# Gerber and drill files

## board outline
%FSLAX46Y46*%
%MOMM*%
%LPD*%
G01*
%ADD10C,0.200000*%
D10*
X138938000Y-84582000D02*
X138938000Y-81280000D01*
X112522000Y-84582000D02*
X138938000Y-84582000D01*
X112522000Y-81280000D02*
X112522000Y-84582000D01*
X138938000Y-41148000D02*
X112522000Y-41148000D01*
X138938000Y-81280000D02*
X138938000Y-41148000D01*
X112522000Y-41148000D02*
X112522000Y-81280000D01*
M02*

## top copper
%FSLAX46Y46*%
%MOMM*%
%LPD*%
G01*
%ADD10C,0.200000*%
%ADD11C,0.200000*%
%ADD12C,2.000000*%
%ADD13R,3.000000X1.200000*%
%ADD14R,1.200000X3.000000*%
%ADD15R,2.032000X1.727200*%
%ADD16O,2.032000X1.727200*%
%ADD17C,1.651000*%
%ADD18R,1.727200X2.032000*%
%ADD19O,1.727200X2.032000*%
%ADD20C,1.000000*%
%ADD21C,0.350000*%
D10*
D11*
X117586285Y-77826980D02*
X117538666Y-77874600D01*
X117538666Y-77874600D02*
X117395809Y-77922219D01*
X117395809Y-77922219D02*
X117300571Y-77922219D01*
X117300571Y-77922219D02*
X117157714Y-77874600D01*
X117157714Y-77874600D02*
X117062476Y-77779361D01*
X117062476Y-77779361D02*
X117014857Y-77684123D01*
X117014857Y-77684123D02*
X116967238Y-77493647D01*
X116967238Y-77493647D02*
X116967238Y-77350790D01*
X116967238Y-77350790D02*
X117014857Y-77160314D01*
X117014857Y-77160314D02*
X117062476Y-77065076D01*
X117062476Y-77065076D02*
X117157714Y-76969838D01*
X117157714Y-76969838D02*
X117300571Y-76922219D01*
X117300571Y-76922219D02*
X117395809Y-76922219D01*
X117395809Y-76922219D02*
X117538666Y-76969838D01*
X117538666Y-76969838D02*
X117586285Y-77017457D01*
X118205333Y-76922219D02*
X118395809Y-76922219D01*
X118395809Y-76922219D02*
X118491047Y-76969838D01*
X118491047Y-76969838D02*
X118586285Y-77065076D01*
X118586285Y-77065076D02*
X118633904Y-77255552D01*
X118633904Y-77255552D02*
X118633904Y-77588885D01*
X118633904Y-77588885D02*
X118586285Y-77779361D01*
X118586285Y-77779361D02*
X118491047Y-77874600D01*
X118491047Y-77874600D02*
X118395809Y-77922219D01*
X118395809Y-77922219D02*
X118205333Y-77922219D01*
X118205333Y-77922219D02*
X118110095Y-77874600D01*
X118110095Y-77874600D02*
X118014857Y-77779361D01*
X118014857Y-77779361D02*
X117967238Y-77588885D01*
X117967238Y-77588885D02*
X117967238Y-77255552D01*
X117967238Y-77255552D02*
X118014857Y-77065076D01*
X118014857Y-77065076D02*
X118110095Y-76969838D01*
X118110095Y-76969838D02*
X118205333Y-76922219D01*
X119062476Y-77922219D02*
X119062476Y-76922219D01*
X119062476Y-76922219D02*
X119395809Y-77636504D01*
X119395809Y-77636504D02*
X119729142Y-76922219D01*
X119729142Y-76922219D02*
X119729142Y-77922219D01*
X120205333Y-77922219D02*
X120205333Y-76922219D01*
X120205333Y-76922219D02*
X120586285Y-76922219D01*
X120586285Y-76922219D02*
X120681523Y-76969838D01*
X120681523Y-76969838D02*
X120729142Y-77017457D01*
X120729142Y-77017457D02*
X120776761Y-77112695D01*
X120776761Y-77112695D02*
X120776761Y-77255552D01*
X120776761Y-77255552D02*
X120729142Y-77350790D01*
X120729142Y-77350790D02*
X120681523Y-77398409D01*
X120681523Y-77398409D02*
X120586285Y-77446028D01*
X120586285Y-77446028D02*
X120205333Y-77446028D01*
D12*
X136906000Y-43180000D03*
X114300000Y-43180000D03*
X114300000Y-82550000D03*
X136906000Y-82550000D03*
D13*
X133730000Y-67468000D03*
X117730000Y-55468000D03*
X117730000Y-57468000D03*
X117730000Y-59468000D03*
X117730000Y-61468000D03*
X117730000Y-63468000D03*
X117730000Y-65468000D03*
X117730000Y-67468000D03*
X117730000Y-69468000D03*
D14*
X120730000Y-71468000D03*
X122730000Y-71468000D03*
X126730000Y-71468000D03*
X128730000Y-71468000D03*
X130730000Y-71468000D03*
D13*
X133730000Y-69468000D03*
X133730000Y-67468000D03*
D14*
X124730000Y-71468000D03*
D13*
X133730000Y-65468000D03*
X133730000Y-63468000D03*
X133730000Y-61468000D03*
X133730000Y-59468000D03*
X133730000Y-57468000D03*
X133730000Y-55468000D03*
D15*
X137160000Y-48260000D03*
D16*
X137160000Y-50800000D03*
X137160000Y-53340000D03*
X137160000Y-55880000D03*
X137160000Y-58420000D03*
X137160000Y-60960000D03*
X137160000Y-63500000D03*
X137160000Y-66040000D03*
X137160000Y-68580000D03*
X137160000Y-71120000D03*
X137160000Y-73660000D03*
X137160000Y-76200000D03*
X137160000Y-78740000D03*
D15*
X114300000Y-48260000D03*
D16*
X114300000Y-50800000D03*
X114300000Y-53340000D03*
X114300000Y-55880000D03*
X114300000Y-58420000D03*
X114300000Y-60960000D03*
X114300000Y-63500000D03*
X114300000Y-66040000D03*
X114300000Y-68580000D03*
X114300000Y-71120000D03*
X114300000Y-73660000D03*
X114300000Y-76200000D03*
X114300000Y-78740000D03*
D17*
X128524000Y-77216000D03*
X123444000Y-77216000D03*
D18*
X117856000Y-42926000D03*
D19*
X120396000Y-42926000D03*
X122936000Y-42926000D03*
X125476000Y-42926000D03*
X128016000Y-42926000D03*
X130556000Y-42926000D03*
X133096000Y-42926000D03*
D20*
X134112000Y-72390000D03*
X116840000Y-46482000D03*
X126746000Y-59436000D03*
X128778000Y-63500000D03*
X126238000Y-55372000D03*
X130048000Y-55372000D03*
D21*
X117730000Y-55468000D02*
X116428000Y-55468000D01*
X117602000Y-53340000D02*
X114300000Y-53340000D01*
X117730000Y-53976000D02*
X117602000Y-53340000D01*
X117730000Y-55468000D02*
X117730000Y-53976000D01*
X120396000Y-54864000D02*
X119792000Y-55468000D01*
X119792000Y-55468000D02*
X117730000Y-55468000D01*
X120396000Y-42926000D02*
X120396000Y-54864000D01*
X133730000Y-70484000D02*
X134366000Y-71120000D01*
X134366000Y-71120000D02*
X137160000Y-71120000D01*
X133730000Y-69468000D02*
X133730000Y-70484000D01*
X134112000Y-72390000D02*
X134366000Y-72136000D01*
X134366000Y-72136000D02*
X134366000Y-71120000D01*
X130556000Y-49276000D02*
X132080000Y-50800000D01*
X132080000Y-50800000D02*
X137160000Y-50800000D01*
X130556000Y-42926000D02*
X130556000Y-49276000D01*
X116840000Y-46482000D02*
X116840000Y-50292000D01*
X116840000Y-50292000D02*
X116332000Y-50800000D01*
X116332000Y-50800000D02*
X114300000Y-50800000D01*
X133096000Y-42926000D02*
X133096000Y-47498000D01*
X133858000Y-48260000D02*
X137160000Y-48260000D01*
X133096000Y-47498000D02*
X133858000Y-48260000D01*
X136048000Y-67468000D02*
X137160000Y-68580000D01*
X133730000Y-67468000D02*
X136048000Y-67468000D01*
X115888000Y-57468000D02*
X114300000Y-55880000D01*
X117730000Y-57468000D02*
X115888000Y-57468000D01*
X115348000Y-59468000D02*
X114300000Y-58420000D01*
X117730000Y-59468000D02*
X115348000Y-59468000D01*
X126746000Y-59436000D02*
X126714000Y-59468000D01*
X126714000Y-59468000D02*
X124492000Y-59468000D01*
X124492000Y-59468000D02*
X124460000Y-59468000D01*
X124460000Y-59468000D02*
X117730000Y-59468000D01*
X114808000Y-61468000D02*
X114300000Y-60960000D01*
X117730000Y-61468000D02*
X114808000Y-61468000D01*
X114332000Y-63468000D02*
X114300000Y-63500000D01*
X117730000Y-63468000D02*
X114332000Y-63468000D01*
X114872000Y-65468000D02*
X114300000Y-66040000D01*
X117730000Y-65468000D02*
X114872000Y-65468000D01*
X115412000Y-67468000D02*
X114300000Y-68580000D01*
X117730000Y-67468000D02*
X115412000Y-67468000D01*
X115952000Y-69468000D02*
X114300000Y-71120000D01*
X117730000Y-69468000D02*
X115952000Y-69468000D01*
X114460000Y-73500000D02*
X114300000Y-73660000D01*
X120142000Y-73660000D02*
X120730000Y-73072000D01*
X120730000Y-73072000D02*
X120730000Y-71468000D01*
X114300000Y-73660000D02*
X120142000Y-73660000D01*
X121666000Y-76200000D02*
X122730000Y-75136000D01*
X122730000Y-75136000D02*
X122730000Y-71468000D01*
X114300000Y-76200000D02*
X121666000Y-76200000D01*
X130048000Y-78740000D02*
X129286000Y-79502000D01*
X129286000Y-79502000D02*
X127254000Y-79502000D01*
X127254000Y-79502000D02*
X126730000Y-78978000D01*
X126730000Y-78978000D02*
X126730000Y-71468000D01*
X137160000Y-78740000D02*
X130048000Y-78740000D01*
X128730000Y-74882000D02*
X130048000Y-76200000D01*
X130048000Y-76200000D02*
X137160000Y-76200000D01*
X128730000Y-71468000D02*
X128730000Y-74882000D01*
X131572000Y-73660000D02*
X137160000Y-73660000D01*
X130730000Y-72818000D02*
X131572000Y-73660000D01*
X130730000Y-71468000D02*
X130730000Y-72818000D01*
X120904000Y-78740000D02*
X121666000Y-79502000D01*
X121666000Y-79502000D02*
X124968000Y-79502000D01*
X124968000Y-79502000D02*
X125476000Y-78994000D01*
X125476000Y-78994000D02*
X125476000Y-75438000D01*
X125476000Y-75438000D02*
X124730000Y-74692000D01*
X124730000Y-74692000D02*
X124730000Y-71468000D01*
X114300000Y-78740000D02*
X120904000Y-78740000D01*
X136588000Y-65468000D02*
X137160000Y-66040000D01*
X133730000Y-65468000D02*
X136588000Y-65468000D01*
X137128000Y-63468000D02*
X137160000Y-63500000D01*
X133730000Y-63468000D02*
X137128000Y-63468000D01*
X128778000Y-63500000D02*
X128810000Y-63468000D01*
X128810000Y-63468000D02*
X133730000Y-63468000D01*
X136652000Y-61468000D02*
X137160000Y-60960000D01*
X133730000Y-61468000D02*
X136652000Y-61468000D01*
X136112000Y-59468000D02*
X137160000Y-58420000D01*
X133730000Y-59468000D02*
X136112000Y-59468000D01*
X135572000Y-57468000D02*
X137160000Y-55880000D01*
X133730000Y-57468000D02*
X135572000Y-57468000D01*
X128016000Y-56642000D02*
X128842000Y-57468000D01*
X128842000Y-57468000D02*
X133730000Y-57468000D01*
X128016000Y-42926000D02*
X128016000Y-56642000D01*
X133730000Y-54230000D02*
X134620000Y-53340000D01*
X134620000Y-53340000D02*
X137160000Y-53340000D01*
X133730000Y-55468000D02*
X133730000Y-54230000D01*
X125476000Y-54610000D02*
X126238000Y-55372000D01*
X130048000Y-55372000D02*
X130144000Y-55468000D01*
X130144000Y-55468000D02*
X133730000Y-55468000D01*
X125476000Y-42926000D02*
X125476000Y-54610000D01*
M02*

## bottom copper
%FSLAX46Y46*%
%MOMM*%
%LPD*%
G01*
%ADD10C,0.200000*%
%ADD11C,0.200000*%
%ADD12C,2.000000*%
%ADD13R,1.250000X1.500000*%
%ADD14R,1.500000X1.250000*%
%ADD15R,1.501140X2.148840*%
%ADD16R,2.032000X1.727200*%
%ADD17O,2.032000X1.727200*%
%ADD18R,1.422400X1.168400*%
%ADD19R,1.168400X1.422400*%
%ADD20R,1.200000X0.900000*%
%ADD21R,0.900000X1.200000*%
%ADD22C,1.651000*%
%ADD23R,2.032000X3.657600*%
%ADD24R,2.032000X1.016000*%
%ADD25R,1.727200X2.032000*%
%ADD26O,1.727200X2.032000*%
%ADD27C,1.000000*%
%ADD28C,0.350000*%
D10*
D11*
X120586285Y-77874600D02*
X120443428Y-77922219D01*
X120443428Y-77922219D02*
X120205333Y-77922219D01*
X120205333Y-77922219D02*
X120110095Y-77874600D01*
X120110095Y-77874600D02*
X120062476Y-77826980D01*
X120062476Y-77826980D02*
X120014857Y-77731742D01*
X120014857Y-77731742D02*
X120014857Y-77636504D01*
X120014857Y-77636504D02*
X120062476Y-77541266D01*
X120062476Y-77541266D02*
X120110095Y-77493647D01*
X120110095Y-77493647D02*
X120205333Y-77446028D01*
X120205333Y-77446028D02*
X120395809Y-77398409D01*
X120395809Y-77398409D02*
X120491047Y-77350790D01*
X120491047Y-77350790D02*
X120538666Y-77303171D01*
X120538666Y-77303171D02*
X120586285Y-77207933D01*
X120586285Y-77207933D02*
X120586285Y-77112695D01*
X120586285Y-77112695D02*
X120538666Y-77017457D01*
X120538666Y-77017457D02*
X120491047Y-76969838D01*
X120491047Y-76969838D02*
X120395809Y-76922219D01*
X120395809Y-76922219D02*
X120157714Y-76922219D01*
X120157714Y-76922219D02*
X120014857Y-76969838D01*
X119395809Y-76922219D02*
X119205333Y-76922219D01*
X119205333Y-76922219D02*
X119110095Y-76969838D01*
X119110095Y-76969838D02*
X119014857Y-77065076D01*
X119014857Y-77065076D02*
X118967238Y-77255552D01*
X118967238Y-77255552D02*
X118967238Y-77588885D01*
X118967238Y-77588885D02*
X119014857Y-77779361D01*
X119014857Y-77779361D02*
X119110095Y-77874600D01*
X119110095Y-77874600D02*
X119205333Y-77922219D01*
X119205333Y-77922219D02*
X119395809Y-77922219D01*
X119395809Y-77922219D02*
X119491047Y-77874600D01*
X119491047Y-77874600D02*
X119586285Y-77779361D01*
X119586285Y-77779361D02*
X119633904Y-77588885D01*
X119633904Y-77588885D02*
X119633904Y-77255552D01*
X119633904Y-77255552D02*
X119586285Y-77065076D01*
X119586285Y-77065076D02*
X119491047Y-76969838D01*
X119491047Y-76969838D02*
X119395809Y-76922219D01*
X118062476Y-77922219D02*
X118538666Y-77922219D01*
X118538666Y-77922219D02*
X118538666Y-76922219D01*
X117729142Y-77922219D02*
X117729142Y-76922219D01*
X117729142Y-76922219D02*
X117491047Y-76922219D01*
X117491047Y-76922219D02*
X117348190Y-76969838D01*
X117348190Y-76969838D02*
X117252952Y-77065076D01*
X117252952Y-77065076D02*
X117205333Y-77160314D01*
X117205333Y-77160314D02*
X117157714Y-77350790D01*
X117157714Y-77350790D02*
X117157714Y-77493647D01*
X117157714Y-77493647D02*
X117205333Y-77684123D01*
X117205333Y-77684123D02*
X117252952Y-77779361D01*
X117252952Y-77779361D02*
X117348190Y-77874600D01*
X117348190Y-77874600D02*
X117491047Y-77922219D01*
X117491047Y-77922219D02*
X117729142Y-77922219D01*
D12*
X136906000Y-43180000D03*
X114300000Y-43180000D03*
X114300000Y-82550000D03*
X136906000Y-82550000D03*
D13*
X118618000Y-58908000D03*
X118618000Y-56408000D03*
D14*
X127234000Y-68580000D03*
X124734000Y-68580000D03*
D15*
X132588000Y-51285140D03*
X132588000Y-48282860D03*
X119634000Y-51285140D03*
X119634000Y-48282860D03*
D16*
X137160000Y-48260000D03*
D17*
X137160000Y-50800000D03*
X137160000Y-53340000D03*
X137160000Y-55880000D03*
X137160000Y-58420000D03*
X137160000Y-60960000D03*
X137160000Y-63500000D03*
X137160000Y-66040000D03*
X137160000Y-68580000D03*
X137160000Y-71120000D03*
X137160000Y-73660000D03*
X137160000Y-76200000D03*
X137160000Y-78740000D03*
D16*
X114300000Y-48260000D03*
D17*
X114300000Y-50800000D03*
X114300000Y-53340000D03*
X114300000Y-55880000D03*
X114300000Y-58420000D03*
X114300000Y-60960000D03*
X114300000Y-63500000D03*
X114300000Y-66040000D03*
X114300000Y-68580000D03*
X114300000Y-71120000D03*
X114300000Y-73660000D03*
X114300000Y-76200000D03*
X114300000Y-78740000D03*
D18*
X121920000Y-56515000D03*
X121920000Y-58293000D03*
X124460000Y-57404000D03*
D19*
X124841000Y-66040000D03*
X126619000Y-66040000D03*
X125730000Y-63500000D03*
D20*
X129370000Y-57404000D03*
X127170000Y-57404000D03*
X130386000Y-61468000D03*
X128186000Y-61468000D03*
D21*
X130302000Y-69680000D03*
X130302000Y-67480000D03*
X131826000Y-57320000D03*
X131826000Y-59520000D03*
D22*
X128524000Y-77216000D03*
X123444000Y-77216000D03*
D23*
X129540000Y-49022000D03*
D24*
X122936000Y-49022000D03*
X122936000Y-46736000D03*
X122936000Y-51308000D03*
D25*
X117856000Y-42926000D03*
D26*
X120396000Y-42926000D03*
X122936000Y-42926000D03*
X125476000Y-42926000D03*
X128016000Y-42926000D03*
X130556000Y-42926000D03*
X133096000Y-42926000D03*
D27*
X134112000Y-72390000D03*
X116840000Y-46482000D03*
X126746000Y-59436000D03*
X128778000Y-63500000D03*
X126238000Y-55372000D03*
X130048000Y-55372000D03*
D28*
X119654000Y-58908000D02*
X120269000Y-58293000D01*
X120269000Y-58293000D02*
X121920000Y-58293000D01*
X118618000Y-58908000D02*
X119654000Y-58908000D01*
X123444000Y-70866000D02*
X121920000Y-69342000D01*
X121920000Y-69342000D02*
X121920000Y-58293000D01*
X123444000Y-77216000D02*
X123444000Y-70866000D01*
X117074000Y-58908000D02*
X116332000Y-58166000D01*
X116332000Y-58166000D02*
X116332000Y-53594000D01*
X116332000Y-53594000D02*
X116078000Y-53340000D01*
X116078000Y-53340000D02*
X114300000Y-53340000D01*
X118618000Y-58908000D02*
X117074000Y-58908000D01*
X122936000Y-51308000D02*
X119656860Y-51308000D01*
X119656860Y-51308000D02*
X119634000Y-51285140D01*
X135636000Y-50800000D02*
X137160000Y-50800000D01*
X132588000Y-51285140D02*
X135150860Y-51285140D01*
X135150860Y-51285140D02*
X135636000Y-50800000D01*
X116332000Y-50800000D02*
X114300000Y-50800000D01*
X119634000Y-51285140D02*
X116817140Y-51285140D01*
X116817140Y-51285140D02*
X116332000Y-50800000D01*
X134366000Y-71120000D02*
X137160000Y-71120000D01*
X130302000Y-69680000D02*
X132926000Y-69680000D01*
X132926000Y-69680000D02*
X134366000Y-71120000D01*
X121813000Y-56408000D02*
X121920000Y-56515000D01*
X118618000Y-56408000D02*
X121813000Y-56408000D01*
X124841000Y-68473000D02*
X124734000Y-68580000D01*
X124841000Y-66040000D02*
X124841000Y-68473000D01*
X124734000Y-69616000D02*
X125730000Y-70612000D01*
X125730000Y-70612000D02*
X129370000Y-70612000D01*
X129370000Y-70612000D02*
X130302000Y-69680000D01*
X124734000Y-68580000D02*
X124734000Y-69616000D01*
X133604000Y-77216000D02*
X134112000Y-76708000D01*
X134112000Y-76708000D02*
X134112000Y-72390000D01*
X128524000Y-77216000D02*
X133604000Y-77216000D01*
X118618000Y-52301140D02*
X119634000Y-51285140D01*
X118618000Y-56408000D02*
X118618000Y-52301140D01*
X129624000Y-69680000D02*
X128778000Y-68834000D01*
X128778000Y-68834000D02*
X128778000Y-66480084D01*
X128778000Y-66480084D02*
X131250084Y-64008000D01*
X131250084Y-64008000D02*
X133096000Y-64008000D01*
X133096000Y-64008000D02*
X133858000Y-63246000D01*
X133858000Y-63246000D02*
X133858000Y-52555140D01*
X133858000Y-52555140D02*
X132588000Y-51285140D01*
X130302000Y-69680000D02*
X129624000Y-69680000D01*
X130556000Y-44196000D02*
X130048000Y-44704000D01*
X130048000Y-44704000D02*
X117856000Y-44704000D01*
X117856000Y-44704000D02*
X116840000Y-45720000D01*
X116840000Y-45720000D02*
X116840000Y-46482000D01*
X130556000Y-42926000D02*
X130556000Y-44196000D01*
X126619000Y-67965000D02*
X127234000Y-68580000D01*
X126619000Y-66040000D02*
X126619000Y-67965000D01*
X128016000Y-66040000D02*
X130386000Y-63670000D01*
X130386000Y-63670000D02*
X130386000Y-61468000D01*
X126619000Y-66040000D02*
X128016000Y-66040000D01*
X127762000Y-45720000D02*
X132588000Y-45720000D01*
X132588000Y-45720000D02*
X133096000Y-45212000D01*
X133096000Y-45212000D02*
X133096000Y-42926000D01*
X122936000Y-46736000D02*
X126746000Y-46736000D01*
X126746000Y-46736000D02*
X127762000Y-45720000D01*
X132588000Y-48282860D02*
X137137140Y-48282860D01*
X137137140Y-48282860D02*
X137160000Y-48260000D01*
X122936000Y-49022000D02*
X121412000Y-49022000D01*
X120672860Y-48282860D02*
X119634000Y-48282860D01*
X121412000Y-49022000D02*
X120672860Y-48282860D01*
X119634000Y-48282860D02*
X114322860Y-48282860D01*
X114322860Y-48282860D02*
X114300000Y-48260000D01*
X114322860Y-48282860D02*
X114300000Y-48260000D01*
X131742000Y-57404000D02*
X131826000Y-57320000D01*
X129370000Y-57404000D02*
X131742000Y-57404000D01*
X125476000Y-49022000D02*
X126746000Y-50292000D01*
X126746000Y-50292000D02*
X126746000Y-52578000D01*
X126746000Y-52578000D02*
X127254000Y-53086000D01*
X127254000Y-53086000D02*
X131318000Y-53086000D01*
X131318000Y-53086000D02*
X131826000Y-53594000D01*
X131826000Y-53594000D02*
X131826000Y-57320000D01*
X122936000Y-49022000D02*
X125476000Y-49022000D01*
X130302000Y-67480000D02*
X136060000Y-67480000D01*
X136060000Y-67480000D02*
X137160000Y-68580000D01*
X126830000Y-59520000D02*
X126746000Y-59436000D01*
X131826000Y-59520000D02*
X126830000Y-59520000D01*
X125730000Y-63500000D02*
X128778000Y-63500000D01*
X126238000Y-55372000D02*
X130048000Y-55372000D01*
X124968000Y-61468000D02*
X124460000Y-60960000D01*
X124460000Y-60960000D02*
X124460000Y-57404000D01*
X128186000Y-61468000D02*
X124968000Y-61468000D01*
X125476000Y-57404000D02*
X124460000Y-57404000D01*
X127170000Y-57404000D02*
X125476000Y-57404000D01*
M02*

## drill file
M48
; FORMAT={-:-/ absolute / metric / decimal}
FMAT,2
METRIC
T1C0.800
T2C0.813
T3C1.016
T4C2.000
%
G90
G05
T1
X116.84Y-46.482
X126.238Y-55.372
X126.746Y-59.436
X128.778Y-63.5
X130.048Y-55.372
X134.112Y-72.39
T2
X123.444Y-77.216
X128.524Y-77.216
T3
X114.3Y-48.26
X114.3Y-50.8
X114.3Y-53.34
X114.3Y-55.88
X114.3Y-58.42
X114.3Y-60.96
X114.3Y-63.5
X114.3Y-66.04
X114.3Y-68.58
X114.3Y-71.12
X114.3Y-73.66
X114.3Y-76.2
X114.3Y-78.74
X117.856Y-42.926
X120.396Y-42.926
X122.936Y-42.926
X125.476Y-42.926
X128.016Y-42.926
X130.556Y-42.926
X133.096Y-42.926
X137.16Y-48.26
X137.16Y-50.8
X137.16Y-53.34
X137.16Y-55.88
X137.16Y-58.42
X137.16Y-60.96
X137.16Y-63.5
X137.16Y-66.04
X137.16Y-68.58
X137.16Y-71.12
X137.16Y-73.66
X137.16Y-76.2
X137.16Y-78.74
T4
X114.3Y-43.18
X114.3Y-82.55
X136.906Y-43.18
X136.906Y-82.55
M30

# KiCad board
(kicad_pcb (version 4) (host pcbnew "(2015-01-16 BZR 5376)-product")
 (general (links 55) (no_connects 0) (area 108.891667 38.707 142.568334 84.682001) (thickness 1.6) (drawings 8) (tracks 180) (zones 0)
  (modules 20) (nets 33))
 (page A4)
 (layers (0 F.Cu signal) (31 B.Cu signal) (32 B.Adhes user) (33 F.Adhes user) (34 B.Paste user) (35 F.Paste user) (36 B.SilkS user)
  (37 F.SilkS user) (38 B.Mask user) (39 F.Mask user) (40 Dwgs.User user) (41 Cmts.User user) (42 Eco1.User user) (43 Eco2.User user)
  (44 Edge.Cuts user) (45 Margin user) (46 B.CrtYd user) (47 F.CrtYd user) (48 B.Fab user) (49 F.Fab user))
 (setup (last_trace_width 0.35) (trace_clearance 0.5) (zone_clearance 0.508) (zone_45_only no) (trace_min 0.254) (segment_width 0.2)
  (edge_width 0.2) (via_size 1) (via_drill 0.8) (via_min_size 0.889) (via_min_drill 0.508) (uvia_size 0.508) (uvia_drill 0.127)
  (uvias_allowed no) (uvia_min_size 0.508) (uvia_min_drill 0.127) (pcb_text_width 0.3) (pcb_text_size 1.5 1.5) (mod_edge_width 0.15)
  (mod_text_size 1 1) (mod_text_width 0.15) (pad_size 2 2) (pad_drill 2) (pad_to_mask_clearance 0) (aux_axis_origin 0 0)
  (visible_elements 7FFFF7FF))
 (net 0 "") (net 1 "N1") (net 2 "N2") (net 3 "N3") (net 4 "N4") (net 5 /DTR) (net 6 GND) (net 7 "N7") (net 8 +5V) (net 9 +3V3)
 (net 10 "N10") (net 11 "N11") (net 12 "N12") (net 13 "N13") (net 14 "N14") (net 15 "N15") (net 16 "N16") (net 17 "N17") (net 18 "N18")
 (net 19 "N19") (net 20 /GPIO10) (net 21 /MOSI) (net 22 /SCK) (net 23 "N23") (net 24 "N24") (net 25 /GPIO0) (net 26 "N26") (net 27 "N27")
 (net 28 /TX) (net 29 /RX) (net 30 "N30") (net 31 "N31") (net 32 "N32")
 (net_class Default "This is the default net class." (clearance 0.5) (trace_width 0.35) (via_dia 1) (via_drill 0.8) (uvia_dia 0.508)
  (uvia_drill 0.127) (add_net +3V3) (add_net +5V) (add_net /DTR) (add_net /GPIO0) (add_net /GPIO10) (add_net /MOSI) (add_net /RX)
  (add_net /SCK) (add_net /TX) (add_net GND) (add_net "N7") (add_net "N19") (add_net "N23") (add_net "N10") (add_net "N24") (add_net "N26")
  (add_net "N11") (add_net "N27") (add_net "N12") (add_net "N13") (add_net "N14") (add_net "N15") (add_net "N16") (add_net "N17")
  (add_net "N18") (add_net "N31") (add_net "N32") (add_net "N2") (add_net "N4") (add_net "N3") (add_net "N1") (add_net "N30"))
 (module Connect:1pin (layer F.Cu) (at 136.906 43.18)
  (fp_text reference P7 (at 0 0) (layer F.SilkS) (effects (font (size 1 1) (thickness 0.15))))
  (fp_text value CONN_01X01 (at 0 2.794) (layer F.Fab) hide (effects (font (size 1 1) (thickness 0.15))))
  (pad 1 thru_hole circle (at 0 0) (size 2 2) (drill 2) (layers *.Cu *.Mask F.SilkS) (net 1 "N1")))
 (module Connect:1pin (layer F.Cu) (at 114.3 43.18)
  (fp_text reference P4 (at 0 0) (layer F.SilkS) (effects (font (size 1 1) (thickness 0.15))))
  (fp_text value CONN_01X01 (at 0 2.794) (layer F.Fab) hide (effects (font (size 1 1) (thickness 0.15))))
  (pad 1 thru_hole circle (at 0 0) (size 2 2) (drill 2) (layers *.Cu *.Mask F.SilkS) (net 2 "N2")))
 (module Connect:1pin (layer F.Cu) (at 114.3 82.55)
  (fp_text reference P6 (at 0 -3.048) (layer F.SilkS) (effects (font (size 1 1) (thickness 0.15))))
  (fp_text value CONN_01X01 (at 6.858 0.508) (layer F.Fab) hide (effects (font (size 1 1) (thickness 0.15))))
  (pad 1 thru_hole circle (at 0 0) (size 2 2) (drill 2) (layers *.Cu *.Mask F.SilkS) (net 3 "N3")))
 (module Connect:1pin (layer F.Cu) (at 136.906 82.55)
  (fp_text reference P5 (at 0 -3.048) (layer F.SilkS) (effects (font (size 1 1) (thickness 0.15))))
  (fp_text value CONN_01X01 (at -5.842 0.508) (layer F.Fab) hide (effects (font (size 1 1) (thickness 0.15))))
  (pad 1 thru_hole circle (at 0 0) (size 2 2) (drill 2) (layers *.Cu *.Mask F.SilkS) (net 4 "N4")))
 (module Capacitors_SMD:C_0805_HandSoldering (layer B.Cu) (at 118.618 57.658 90)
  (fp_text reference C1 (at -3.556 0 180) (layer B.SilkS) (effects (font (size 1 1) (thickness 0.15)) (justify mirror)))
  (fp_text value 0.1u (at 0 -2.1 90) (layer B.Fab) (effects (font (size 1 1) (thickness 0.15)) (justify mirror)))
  (pad 1 smd rect (at -1.25 0 90) (size 1.5 1.25) (layers B.Cu B.Paste B.Mask) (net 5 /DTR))
  (pad 2 smd rect (at 1.25 0 90) (size 1.5 1.25) (layers B.Cu B.Paste B.Mask) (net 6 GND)))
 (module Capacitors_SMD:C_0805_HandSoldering (layer B.Cu) (at 125.984 68.58 180)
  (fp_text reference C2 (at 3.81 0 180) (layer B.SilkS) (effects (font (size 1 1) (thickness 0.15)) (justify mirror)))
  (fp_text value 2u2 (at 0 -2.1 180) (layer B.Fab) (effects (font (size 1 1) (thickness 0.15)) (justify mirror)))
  (pad 1 smd rect (at -1.25 0 180) (size 1.5 1.25) (layers B.Cu B.Paste B.Mask) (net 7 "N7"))
  (pad 2 smd rect (at 1.25 0 180) (size 1.5 1.25) (layers B.Cu B.Paste B.Mask) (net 6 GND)))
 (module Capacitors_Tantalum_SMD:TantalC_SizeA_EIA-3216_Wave (layer B.Cu) (at 132.588 49.784 270)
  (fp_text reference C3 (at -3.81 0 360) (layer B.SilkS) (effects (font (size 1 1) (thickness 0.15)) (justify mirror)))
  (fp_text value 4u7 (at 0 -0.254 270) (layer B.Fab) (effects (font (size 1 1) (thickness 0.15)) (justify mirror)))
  (pad 2 smd rect (at 1.50114 0 270) (size 2.14884 1.50114) (layers B.Cu B.Paste B.Mask) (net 6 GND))
  (pad 1 smd rect (at -1.50114 0 270) (size 2.14884 1.50114) (layers B.Cu B.Paste B.Mask) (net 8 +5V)))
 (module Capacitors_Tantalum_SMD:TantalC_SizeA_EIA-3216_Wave (layer B.Cu) (at 119.634 49.784 270)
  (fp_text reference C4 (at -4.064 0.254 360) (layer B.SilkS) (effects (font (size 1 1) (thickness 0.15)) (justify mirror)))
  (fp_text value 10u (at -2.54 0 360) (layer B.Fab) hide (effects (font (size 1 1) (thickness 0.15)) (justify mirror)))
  (pad 2 smd rect (at 1.50114 0 270) (size 2.14884 1.50114) (layers B.Cu B.Paste B.Mask) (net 6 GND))
  (pad 1 smd rect (at -1.50114 0 270) (size 2.14884 1.50114) (layers B.Cu B.Paste B.Mask) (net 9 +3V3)))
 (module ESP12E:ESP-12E (layer F.Cu) (at 125.73 61.468 270)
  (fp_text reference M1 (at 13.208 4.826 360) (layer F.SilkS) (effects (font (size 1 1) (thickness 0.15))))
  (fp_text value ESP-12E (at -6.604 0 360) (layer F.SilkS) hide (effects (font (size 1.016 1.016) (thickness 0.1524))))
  (pad 16 smd rect (at 6 -8 270) (size 1.2 3) (layers F.Cu F.Paste F.Mask) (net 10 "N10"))
  (pad 1 smd rect (at -6 8 270) (size 1.2 3) (layers F.Cu F.Paste F.Mask) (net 5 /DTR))
  (pad 2 smd rect (at -4 8 270) (size 1.2 3) (layers F.Cu F.Paste F.Mask) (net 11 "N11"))
  (pad 3 smd rect (at -2 8 270) (size 1.2 3) (layers F.Cu F.Paste F.Mask) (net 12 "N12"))
  (pad 4 smd rect (at 0 8 270) (size 1.2 3) (layers F.Cu F.Paste F.Mask) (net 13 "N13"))
  (pad 5 smd rect (at 2 8 270) (size 1.2 3) (layers F.Cu F.Paste F.Mask) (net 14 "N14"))
  (pad 6 smd rect (at 4 8 270) (size 1.2 3) (layers F.Cu F.Paste F.Mask) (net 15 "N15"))
  (pad 7 smd rect (at 6 8 270) (size 1.2 3) (layers F.Cu F.Paste F.Mask) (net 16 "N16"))
  (pad 8 smd rect (at 8 8 270) (size 1.2 3) (layers F.Cu F.Paste F.Mask) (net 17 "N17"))
  (pad 9 smd rect (at 10 5 180) (size 1.2 3) (layers F.Cu F.Paste F.Mask) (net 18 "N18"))
  (pad 10 smd rect (at 10 3 180) (size 1.2 3) (layers F.Cu F.Paste F.Mask) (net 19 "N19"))
  (pad 12 smd rect (at 10 -1 180) (size 1.2 3) (layers F.Cu F.Paste F.Mask) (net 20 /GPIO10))
  (pad 13 smd rect (at 10 -3 180) (size 1.2 3) (layers F.Cu F.Paste F.Mask) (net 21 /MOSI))
  (pad 14 smd rect (at 10 -5 180) (size 1.2 3) (layers F.Cu F.Paste F.Mask) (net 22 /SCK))
  (pad 15 smd rect (at 8 -8 270) (size 1.2 3) (layers F.Cu F.Paste F.Mask) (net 6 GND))
  (pad 16 smd rect (at 6 -8 270) (size 1.2 3) (layers F.Cu F.Paste F.Mask) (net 10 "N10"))
  (pad 11 smd rect (at 10 1 180) (size 1.2 3) (layers F.Cu F.Paste F.Mask) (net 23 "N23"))
  (pad 17 smd rect (at 4 -8 270) (size 1.2 3) (layers F.Cu F.Paste F.Mask) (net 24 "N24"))
  (pad 18 smd rect (at 2 -8 270) (size 1.2 3) (layers F.Cu F.Paste F.Mask) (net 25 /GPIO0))
  (pad 19 smd rect (at 0 -8 270) (size 1.2 3) (layers F.Cu F.Paste F.Mask) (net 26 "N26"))
  (pad 20 smd rect (at -2 -8 270) (size 1.2 3) (layers F.Cu F.Paste F.Mask) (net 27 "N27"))
  (pad 21 smd rect (at -4 -8 270) (size 1.2 3) (layers F.Cu F.Paste F.Mask) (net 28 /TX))
  (pad 22 smd rect (at -6 -8 270) (size 1.2 3) (layers F.Cu F.Paste F.Mask) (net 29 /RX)))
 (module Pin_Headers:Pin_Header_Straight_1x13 (layer F.Cu) (at 137.16 48.26)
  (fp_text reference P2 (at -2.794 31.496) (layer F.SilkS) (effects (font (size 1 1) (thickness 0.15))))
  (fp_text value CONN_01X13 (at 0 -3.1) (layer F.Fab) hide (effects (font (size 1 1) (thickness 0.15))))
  (pad 1 thru_hole rect (at 0 0) (size 2.032 1.7272) (drill 1.016) (layers *.Cu *.Mask F.SilkS) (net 8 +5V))
  (pad 2 thru_hole oval (at 0 2.54) (size 2.032 1.7272) (drill 1.016) (layers *.Cu *.Mask F.SilkS) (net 6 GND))
  (pad 3 thru_hole oval (at 0 5.08) (size 2.032 1.7272) (drill 1.016) (layers *.Cu *.Mask F.SilkS) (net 29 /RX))
  (pad 4 thru_hole oval (at 0 7.62) (size 2.032 1.7272) (drill 1.016) (layers *.Cu *.Mask F.SilkS) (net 28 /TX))
  (pad 5 thru_hole oval (at 0 10.16) (size 2.032 1.7272) (drill 1.016) (layers *.Cu *.Mask F.SilkS) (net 27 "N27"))
  (pad 6 thru_hole oval (at 0 12.7) (size 2.032 1.7272) (drill 1.016) (layers *.Cu *.Mask F.SilkS) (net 26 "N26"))
  (pad 7 thru_hole oval (at 0 15.24) (size 2.032 1.7272) (drill 1.016) (layers *.Cu *.Mask F.SilkS) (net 25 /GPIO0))
  (pad 8 thru_hole oval (at 0 17.78) (size 2.032 1.7272) (drill 1.016) (layers *.Cu *.Mask F.SilkS) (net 24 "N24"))
  (pad 9 thru_hole oval (at 0 20.32) (size 2.032 1.7272) (drill 1.016) (layers *.Cu *.Mask F.SilkS) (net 10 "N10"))
  (pad 10 thru_hole oval (at 0 22.86) (size 2.032 1.7272) (drill 1.016) (layers *.Cu *.Mask F.SilkS) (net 6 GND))
  (pad 11 thru_hole oval (at 0 25.4) (size 2.032 1.7272) (drill 1.016) (layers *.Cu *.Mask F.SilkS) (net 22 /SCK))
  (pad 12 thru_hole oval (at 0 27.94) (size 2.032 1.7272) (drill 1.016) (layers *.Cu *.Mask F.SilkS) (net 21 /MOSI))
  (pad 13 thru_hole oval (at 0 30.48) (size 2.032 1.7272) (drill 1.016) (layers *.Cu *.Mask F.SilkS) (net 20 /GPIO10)))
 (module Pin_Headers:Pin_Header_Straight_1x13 (layer F.Cu) (at 114.3 48.26)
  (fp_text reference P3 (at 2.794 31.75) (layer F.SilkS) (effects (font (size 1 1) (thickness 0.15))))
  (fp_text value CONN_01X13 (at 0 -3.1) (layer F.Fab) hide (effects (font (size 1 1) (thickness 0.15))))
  (pad 1 thru_hole rect (at 0 0) (size 2.032 1.7272) (drill 1.016) (layers *.Cu *.Mask F.SilkS) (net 9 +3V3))
  (pad 2 thru_hole oval (at 0 2.54) (size 2.032 1.7272) (drill 1.016) (layers *.Cu *.Mask F.SilkS) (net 6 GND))
  (pad 3 thru_hole oval (at 0 5.08) (size 2.032 1.7272) (drill 1.016) (layers *.Cu *.Mask F.SilkS) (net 5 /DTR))
  (pad 4 thru_hole oval (at 0 7.62) (size 2.032 1.7272) (drill 1.016) (layers *.Cu *.Mask F.SilkS) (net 11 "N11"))
  (pad 5 thru_hole oval (at 0 10.16) (size 2.032 1.7272) (drill 1.016) (layers *.Cu *.Mask F.SilkS) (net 12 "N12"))
  (pad 6 thru_hole oval (at 0 12.7) (size 2.032 1.7272) (drill 1.016) (layers *.Cu *.Mask F.SilkS) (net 13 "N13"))
  (pad 7 thru_hole oval (at 0 15.24) (size 2.032 1.7272) (drill 1.016) (layers *.Cu *.Mask F.SilkS) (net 14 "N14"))
  (pad 8 thru_hole oval (at 0 17.78) (size 2.032 1.7272) (drill 1.016) (layers *.Cu *.Mask F.SilkS) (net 15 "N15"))
  (pad 9 thru_hole oval (at 0 20.32) (size 2.032 1.7272) (drill 1.016) (layers *.Cu *.Mask F.SilkS) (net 16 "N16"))
  (pad 10 thru_hole oval (at 0 22.86) (size 2.032 1.7272) (drill 1.016) (layers *.Cu *.Mask F.SilkS) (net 17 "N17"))
  (pad 11 thru_hole oval (at 0 25.4) (size 2.032 1.7272) (drill 1.016) (layers *.Cu *.Mask F.SilkS) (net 18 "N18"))
  (pad 12 thru_hole oval (at 0 27.94) (size 2.032 1.7272) (drill 1.016) (layers *.Cu *.Mask F.SilkS) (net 19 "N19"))
  (pad 13 thru_hole oval (at 0 30.48) (size 2.032 1.7272) (drill 1.016) (layers *.Cu *.Mask F.SilkS) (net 23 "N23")))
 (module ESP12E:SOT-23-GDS (layer B.Cu) (at 123.19 57.404 270)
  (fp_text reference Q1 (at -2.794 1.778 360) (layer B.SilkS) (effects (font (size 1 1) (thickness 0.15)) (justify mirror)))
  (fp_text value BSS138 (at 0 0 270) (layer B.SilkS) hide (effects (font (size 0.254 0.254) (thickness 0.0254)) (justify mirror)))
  (pad S smd rect (at -0.889 1.27 270) (size 1.1684 1.4224) (layers B.Cu B.Paste B.Mask) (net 6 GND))
  (pad G smd rect (at 0.889 1.27 270) (size 1.1684 1.4224) (layers B.Cu B.Paste B.Mask) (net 5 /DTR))
  (pad D smd rect (at 0 -1.27 270) (size 1.1684 1.4224) (layers B.Cu B.Paste B.Mask) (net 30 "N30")))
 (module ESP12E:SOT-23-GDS (layer B.Cu) (at 125.73 64.77)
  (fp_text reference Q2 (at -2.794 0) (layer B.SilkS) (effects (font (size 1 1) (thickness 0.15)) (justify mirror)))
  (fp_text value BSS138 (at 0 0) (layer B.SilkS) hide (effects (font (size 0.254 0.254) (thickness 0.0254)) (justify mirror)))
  (pad S smd rect (at -0.889 1.27) (size 1.1684 1.4224) (layers B.Cu B.Paste B.Mask) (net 6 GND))
  (pad G smd rect (at 0.889 1.27) (size 1.1684 1.4224) (layers B.Cu B.Paste B.Mask) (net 7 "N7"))
  (pad D smd rect (at 0 -1.27) (size 1.1684 1.4224) (layers B.Cu B.Paste B.Mask) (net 25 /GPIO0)))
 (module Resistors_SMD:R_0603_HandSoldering (layer B.Cu) (at 128.27 57.404 180)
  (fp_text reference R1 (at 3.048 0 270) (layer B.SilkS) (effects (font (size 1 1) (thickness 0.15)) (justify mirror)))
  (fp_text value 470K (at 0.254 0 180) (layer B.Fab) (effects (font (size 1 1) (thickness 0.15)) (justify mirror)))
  (pad 1 smd rect (at -1.1 0 180) (size 1.2 0.9) (layers B.Cu B.Paste B.Mask) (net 9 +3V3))
  (pad 2 smd rect (at 1.1 0 180) (size 1.2 0.9) (layers B.Cu B.Paste B.Mask) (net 30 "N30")))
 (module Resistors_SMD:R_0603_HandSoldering (layer B.Cu) (at 129.286 61.468 180)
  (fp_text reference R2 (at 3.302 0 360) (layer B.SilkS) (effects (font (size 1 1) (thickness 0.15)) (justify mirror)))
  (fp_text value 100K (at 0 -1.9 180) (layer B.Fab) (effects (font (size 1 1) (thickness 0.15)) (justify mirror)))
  (pad 1 smd rect (at -1.1 0 180) (size 1.2 0.9) (layers B.Cu B.Paste B.Mask) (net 7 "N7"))
  (pad 2 smd rect (at 1.1 0 180) (size 1.2 0.9) (layers B.Cu B.Paste B.Mask) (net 30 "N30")))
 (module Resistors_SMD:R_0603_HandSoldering (layer B.Cu) (at 130.302 68.58 90)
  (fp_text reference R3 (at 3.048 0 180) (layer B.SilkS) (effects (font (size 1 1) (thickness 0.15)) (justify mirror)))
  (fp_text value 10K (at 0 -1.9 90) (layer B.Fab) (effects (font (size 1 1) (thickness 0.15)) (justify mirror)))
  (pad 1 smd rect (at -1.1 0 90) (size 1.2 0.9) (layers B.Cu B.Paste B.Mask) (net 6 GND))
  (pad 2 smd rect (at 1.1 0 90) (size 1.2 0.9) (layers B.Cu B.Paste B.Mask) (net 10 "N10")))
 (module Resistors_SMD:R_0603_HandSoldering (layer B.Cu) (at 131.826 58.42 270)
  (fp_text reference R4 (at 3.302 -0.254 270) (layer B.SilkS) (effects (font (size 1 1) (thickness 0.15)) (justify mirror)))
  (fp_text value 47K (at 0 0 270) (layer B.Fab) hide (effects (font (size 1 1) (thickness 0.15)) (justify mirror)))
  (pad 1 smd rect (at -1.1 0 270) (size 1.2 0.9) (layers B.Cu B.Paste B.Mask) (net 9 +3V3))
  (pad 2 smd rect (at 1.1 0 270) (size 1.2 0.9) (layers B.Cu B.Paste B.Mask) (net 12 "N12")))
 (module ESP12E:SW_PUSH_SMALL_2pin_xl (layer F.Cu) (at 125.984 77.216 180)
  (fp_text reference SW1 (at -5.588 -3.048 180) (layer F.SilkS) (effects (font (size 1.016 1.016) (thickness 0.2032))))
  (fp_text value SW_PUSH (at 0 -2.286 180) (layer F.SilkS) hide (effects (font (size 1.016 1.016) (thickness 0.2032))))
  (pad 1 thru_hole circle (at -2.54 0 180) (size 1.651 1.651) (drill 0.8128) (layers *.Cu *.Mask F.SilkS) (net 6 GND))
  (pad 2 thru_hole circle (at 2.54 0 180) (size 1.651 1.651) (drill 0.8128) (layers *.Cu *.Mask F.SilkS) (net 5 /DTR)))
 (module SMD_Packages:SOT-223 (layer B.Cu) (at 126.238 49.022 90)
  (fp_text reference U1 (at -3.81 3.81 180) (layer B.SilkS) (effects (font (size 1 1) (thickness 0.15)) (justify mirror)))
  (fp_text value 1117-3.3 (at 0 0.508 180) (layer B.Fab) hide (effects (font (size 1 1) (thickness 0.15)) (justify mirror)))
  (pad 4 smd rect (at 0 3.302 90) (size 3.6576 2.032) (layers B.Cu B.Paste B.Mask))
  (pad 2 smd rect (at 0 -3.302 90) (size 1.016 2.032) (layers B.Cu B.Paste B.Mask) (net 9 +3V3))
  (pad 3 smd rect (at 2.286 -3.302 90) (size 1.016 2.032) (layers B.Cu B.Paste B.Mask) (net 8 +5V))
  (pad 1 smd rect (at -2.286 -3.302 90) (size 1.016 2.032) (layers B.Cu B.Paste B.Mask) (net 6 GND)))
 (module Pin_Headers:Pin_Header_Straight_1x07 (layer F.Cu) (at 117.856 42.926 90)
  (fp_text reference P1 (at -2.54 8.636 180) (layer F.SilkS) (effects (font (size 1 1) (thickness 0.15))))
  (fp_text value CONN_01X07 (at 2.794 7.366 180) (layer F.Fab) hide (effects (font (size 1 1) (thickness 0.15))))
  (pad 1 thru_hole rect (at 0 0 90) (size 2.032 1.7272) (drill 1.016) (layers *.Cu *.Mask F.SilkS) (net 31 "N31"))
  (pad 2 thru_hole oval (at 0 2.54 90) (size 2.032 1.7272) (drill 1.016) (layers *.Cu *.Mask F.SilkS) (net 5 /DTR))
  (pad 3 thru_hole oval (at 0 5.08 90) (size 2.032 1.7272) (drill 1.016) (layers *.Cu *.Mask F.SilkS) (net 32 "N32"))
  (pad 4 thru_hole oval (at 0 7.62 90) (size 2.032 1.7272) (drill 1.016) (layers *.Cu *.Mask F.SilkS) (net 29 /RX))
  (pad 5 thru_hole oval (at 0 10.16 90) (size 2.032 1.7272) (drill 1.016) (layers *.Cu *.Mask F.SilkS) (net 28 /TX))
  (pad 6 thru_hole oval (at 0 12.7 90) (size 2.032 1.7272) (drill 1.016) (layers *.Cu *.Mask F.SilkS) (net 6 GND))
  (pad 7 thru_hole oval (at 0 15.24 90) (size 2.032 1.7272) (drill 1.016) (layers *.Cu *.Mask F.SilkS) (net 8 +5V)))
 (gr_line (start 138.938 84.582) (end 138.938 81.28) (angle 90) (layer Edge.Cuts) (width 0.2))
 (gr_line (start 112.522 84.582) (end 138.938 84.582) (angle 90) (layer Edge.Cuts) (width 0.2))
 (gr_line (start 112.522 81.28) (end 112.522 84.582) (angle 90) (layer Edge.Cuts) (width 0.2))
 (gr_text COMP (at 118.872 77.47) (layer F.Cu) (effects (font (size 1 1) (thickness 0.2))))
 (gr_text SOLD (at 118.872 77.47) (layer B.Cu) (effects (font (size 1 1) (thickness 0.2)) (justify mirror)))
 (gr_line (start 138.938 41.148) (end 112.522 41.148) (angle 90) (layer Edge.Cuts) (width 0.2))
 (gr_line (start 138.938 81.28) (end 138.938 41.148) (angle 90) (layer Edge.Cuts) (width 0.2))
 (gr_line (start 112.522 41.148) (end 112.522 81.28) (angle 90) (layer Edge.Cuts) (width 0.2))
 (segment (start 117.73 55.468) (end 116.428 55.468) (width 0.35) (layer F.Cu) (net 5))
 (segment (start 117.602 53.34) (end 114.3 53.34) (width 0.35) (layer F.Cu) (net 5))
 (segment (start 117.73 53.976) (end 117.602 53.34) (width 0.35) (layer F.Cu) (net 5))
 (segment (start 117.73 55.468) (end 117.73 53.976) (width 0.35) (layer F.Cu) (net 5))
 (segment (start 120.396 54.864) (end 119.792 55.468) (width 0.35) (layer F.Cu) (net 5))
 (segment (start 119.792 55.468) (end 117.73 55.468) (width 0.35) (layer F.Cu) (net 5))
 (segment (start 120.396 42.926) (end 120.396 54.864) (width 0.35) (layer F.Cu) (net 5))
 (segment (start 119.654 58.908) (end 120.269 58.293) (width 0.35) (layer B.Cu) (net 5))
 (segment (start 120.269 58.293) (end 121.92 58.293) (width 0.35) (layer B.Cu) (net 5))
 (segment (start 118.618 58.908) (end 119.654 58.908) (width 0.35) (layer B.Cu) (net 5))
 (segment (start 123.444 70.866) (end 121.92 69.342) (width 0.35) (layer B.Cu) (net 5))
 (segment (start 121.92 69.342) (end 121.92 58.293) (width 0.35) (layer B.Cu) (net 5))
 (segment (start 123.444 77.216) (end 123.444 70.866) (width 0.35) (layer B.Cu) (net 5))
 (segment (start 117.074 58.908) (end 116.332 58.166) (width 0.35) (layer B.Cu) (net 5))
 (segment (start 116.332 58.166) (end 116.332 53.594) (width 0.35) (layer B.Cu) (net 5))
 (segment (start 116.332 53.594) (end 116.078 53.34) (width 0.35) (layer B.Cu) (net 5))
 (segment (start 116.078 53.34) (end 114.3 53.34) (width 0.35) (layer B.Cu) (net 5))
 (segment (start 118.618 58.908) (end 117.074 58.908) (width 0.35) (layer B.Cu) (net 5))
 (segment (start 122.936 51.308) (end 119.65686 51.308) (width 0.35) (layer B.Cu) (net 6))
 (segment (start 119.65686 51.308) (end 119.634 51.28514) (width 0.35) (layer B.Cu) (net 6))
 (segment (start 135.636 50.8) (end 137.16 50.8) (width 0.35) (layer B.Cu) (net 6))
 (segment (start 132.588 51.28514) (end 135.15086 51.28514) (width 0.35) (layer B.Cu) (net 6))
 (segment (start 135.15086 51.28514) (end 135.636 50.8) (width 0.35) (layer B.Cu) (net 6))
 (segment (start 116.332 50.8) (end 114.3 50.8) (width 0.35) (layer B.Cu) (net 6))
 (segment (start 119.634 51.28514) (end 116.81714 51.28514) (width 0.35) (layer B.Cu) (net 6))
 (segment (start 116.81714 51.28514) (end 116.332 50.8) (width 0.35) (layer B.Cu) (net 6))
 (segment (start 134.366 71.12) (end 137.16 71.12) (width 0.35) (layer B.Cu) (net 6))
 (segment (start 130.302 69.68) (end 132.926 69.68) (width 0.35) (layer B.Cu) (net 6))
 (segment (start 132.926 69.68) (end 134.366 71.12) (width 0.35) (layer B.Cu) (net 6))
 (segment (start 133.73 70.484) (end 134.366 71.12) (width 0.35) (layer F.Cu) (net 6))
 (segment (start 134.366 71.12) (end 137.16 71.12) (width 0.35) (layer F.Cu) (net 6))
 (segment (start 133.73 69.468) (end 133.73 70.484) (width 0.35) (layer F.Cu) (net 6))
 (via (at 134.112 72.39) (size 1) (layers F.Cu B.Cu) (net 6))
 (segment (start 134.112 72.39) (end 134.366 72.136) (width 0.35) (layer F.Cu) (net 6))
 (segment (start 134.366 72.136) (end 134.366 71.12) (width 0.35) (layer F.Cu) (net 6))
 (segment (start 130.556 49.276) (end 132.08 50.8) (width 0.35) (layer F.Cu) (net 6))
 (segment (start 132.08 50.8) (end 137.16 50.8) (width 0.35) (layer F.Cu) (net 6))
 (segment (start 130.556 42.926) (end 130.556 49.276) (width 0.35) (layer F.Cu) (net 6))
 (segment (start 121.813 56.408) (end 121.92 56.515) (width 0.35) (layer B.Cu) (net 6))
 (segment (start 118.618 56.408) (end 121.813 56.408) (width 0.35) (layer B.Cu) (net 6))
 (segment (start 124.841 68.473) (end 124.734 68.58) (width 0.35) (layer B.Cu) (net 6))
 (segment (start 124.841 66.04) (end 124.841 68.473) (width 0.35) (layer B.Cu) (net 6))
 (segment (start 124.734 69.616) (end 125.73 70.612) (width 0.35) (layer B.Cu) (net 6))
 (segment (start 125.73 70.612) (end 129.37 70.612) (width 0.35) (layer B.Cu) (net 6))
 (segment (start 129.37 70.612) (end 130.302 69.68) (width 0.35) (layer B.Cu) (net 6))
 (segment (start 124.734 68.58) (end 124.734 69.616) (width 0.35) (layer B.Cu) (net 6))
 (segment (start 133.604 77.216) (end 134.112 76.708) (width 0.35) (layer B.Cu) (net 6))
 (segment (start 134.112 76.708) (end 134.112 72.39) (width 0.35) (layer B.Cu) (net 6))
 (segment (start 128.524 77.216) (end 133.604 77.216) (width 0.35) (layer B.Cu) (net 6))
 (segment (start 118.618 52.30114) (end 119.634 51.28514) (width 0.35) (layer B.Cu) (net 6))
 (segment (start 118.618 56.408) (end 118.618 52.30114) (width 0.35) (layer B.Cu) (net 6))
 (segment (start 129.624 69.68) (end 128.778 68.834) (width 0.35) (layer B.Cu) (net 6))
 (segment (start 128.778 68.834) (end 128.778 66.480084) (width 0.35) (layer B.Cu) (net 6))
 (segment (start 128.778 66.480084) (end 131.250084 64.008) (width 0.35) (layer B.Cu) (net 6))
 (segment (start 131.250084 64.008) (end 133.096 64.008) (width 0.35) (layer B.Cu) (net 6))
 (segment (start 133.096 64.008) (end 133.858 63.246) (width 0.35) (layer B.Cu) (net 6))
 (segment (start 133.858 63.246) (end 133.858 52.55514) (width 0.35) (layer B.Cu) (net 6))
 (segment (start 133.858 52.55514) (end 132.588 51.28514) (width 0.35) (layer B.Cu) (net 6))
 (segment (start 130.302 69.68) (end 129.624 69.68) (width 0.35) (layer B.Cu) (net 6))
 (segment (start 130.556 44.196) (end 130.048 44.704) (width 0.35) (layer B.Cu) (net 6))
 (segment (start 130.048 44.704) (end 117.856 44.704) (width 0.35) (layer B.Cu) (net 6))
 (segment (start 117.856 44.704) (end 116.84 45.72) (width 0.35) (layer B.Cu) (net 6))
 (segment (start 116.84 45.72) (end 116.84 46.482) (width 0.35) (layer B.Cu) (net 6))
 (via (at 116.84 46.482) (size 1) (layers F.Cu B.Cu) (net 6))
 (segment (start 116.84 46.482) (end 116.84 50.292) (width 0.35) (layer F.Cu) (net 6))
 (segment (start 116.84 50.292) (end 116.332 50.8) (width 0.35) (layer F.Cu) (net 6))
 (segment (start 116.332 50.8) (end 114.3 50.8) (width 0.35) (layer F.Cu) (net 6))
 (segment (start 130.556 42.926) (end 130.556 44.196) (width 0.35) (layer B.Cu) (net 6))
 (segment (start 126.619 67.965) (end 127.234 68.58) (width 0.35) (layer B.Cu) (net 7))
 (segment (start 126.619 66.04) (end 126.619 67.965) (width 0.35) (layer B.Cu) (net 7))
 (segment (start 128.016 66.04) (end 130.386 63.67) (width 0.35) (layer B.Cu) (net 7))
 (segment (start 130.386 63.67) (end 130.386 61.468) (width 0.35) (layer B.Cu) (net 7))
 (segment (start 126.619 66.04) (end 128.016 66.04) (width 0.35) (layer B.Cu) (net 7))
 (segment (start 133.096 42.926) (end 133.096 47.498) (width 0.35) (layer F.Cu) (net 8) (status 400000))
 (segment (start 133.858 48.26) (end 137.16 48.26) (width 0.35) (layer F.Cu) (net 8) (status 800000))
 (segment (start 133.096 47.498) (end 133.858 48.26) (width 0.35) (layer F.Cu) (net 8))
 (segment (start 127.762 45.72) (end 132.588 45.72) (width 0.35) (layer B.Cu) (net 8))
 (segment (start 132.588 45.72) (end 133.096 45.212) (width 0.35) (layer B.Cu) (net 8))
 (segment (start 133.096 45.212) (end 133.096 42.926) (width 0.35) (layer B.Cu) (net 8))
 (segment (start 122.936 46.736) (end 126.746 46.736) (width 0.35) (layer B.Cu) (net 8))
 (segment (start 126.746 46.736) (end 127.762 45.72) (width 0.35) (layer B.Cu) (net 8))
 (segment (start 132.588 48.28286) (end 137.13714 48.28286) (width 0.35) (layer B.Cu) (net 8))
 (segment (start 137.13714 48.28286) (end 137.16 48.26) (width 0.35) (layer B.Cu) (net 8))
 (segment (start 122.936 49.022) (end 121.412 49.022) (width 0.35) (layer B.Cu) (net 9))
 (segment (start 120.67286 48.28286) (end 119.634 48.28286) (width 0.35) (layer B.Cu) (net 9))
 (segment (start 121.412 49.022) (end 120.67286 48.28286) (width 0.35) (layer B.Cu) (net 9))
 (segment (start 119.634 48.28286) (end 114.32286 48.28286) (width 0.35) (layer B.Cu) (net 9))
 (segment (start 114.32286 48.28286) (end 114.3 48.26) (width 0.35) (layer B.Cu) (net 9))
 (segment (start 114.32286 48.28286) (end 114.3 48.26) (width 0.35) (layer B.Cu) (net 9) (status 30))
 (segment (start 131.742 57.404) (end 131.826 57.32) (width 0.35) (layer B.Cu) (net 9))
 (segment (start 129.37 57.404) (end 131.742 57.404) (width 0.35) (layer B.Cu) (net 9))
 (segment (start 125.476 49.022) (end 126.746 50.292) (width 0.35) (layer B.Cu) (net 9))
 (segment (start 126.746 50.292) (end 126.746 52.578) (width 0.35) (layer B.Cu) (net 9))
 (segment (start 126.746 52.578) (end 127.254 53.086) (width 0.35) (layer B.Cu) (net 9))
 (segment (start 127.254 53.086) (end 131.318 53.086) (width 0.35) (layer B.Cu) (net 9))
 (segment (start 131.318 53.086) (end 131.826 53.594) (width 0.35) (layer B.Cu) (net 9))
 (segment (start 131.826 53.594) (end 131.826 57.32) (width 0.35) (layer B.Cu) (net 9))
 (segment (start 122.936 49.022) (end 125.476 49.022) (width 0.35) (layer B.Cu) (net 9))
 (segment (start 130.302 67.48) (end 136.06 67.48) (width 0.35) (layer B.Cu) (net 10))
 (segment (start 136.06 67.48) (end 137.16 68.58) (width 0.35) (layer B.Cu) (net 10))
 (segment (start 136.048 67.468) (end 137.16 68.58) (width 0.35) (layer F.Cu) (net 10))
 (segment (start 133.73 67.468) (end 136.048 67.468) (width 0.35) (layer F.Cu) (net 10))
 (segment (start 115.888 57.468) (end 114.3 55.88) (width 0.35) (layer F.Cu) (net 11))
 (segment (start 117.73 57.468) (end 115.888 57.468) (width 0.35) (layer F.Cu) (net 11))
 (segment (start 115.348 59.468) (end 114.3 58.42) (width 0.35) (layer F.Cu) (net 12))
 (segment (start 117.73 59.468) (end 115.348 59.468) (width 0.35) (layer F.Cu) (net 12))
 (segment (start 126.83 59.52) (end 126.746 59.436) (width 0.35) (layer B.Cu) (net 12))
 (via (at 126.746 59.436) (size 1) (layers F.Cu B.Cu) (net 12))
 (segment (start 126.746 59.436) (end 126.714 59.468) (width 0.35) (layer F.Cu) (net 12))
 (segment (start 126.714 59.468) (end 124.492 59.468) (width 0.35) (layer F.Cu) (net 12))
 (segment (start 124.492 59.468) (end 124.46 59.468) (width 0.35) (layer F.Cu) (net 12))
 (segment (start 124.46 59.468) (end 117.73 59.468) (width 0.35) (layer F.Cu) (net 12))
 (segment (start 131.826 59.52) (end 126.83 59.52) (width 0.35) (layer B.Cu) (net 12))
 (segment (start 114.808 61.468) (end 114.3 60.96) (width 0.35) (layer F.Cu) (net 13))
 (segment (start 117.73 61.468) (end 114.808 61.468) (width 0.35) (layer F.Cu) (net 13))
 (segment (start 114.332 63.468) (end 114.3 63.5) (width 0.35) (layer F.Cu) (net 14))
 (segment (start 117.73 63.468) (end 114.332 63.468) (width 0.35) (layer F.Cu) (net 14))
 (segment (start 114.872 65.468) (end 114.3 66.04) (width 0.35) (layer F.Cu) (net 15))
 (segment (start 117.73 65.468) (end 114.872 65.468) (width 0.35) (layer F.Cu) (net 15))
 (segment (start 115.412 67.468) (end 114.3 68.58) (width 0.35) (layer F.Cu) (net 16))
 (segment (start 117.73 67.468) (end 115.412 67.468) (width 0.35) (layer F.Cu) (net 16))
 (segment (start 115.952 69.468) (end 114.3 71.12) (width 0.35) (layer F.Cu) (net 17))
 (segment (start 117.73 69.468) (end 115.952 69.468) (width 0.35) (layer F.Cu) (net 17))
 (segment (start 114.46 73.5) (end 114.3 73.66) (width 0.35) (layer F.Cu) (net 18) (status 30))
 (segment (start 120.142 73.66) (end 120.73 73.072) (width 0.35) (layer F.Cu) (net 18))
 (segment (start 120.73 73.072) (end 120.73 71.468) (width 0.35) (layer F.Cu) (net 18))
 (segment (start 114.3 73.66) (end 120.142 73.66) (width 0.35) (layer F.Cu) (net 18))
 (segment (start 121.666 76.2) (end 122.73 75.136) (width 0.35) (layer F.Cu) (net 19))
 (segment (start 122.73 75.136) (end 122.73 71.468) (width 0.35) (layer F.Cu) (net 19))
 (segment (start 114.3 76.2) (end 121.666 76.2) (width 0.35) (layer F.Cu) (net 19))
 (segment (start 130.048 78.74) (end 129.286 79.502) (width 0.35) (layer F.Cu) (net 20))
 (segment (start 129.286 79.502) (end 127.254 79.502) (width 0.35) (layer F.Cu) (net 20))
 (segment (start 127.254 79.502) (end 126.73 78.978) (width 0.35) (layer F.Cu) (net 20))
 (segment (start 126.73 78.978) (end 126.73 71.468) (width 0.35) (layer F.Cu) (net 20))
 (segment (start 137.16 78.74) (end 130.048 78.74) (width 0.35) (layer F.Cu) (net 20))
 (segment (start 128.73 74.882) (end 130.048 76.2) (width 0.35) (layer F.Cu) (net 21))
 (segment (start 130.048 76.2) (end 137.16 76.2) (width 0.35) (layer F.Cu) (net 21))
 (segment (start 128.73 71.468) (end 128.73 74.882) (width 0.35) (layer F.Cu) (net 21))
 (segment (start 131.572 73.66) (end 137.16 73.66) (width 0.35) (layer F.Cu) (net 22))
 (segment (start 130.73 72.818) (end 131.572 73.66) (width 0.35) (layer F.Cu) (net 22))
 (segment (start 130.73 71.468) (end 130.73 72.818) (width 0.35) (layer F.Cu) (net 22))
 (segment (start 120.904 78.74) (end 121.666 79.502) (width 0.35) (layer F.Cu) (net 23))
 (segment (start 121.666 79.502) (end 124.968 79.502) (width 0.35) (layer F.Cu) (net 23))
 (segment (start 124.968 79.502) (end 125.476 78.994) (width 0.35) (layer F.Cu) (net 23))
 (segment (start 125.476 78.994) (end 125.476 75.438) (width 0.35) (layer F.Cu) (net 23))
 (segment (start 125.476 75.438) (end 124.73 74.692) (width 0.35) (layer F.Cu) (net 23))
 (segment (start 124.73 74.692) (end 124.73 71.468) (width 0.35) (layer F.Cu) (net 23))
 (segment (start 114.3 78.74) (end 120.904 78.74) (width 0.35) (layer F.Cu) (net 23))
 (segment (start 136.588 65.468) (end 137.16 66.04) (width 0.35) (layer F.Cu) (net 24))
 (segment (start 133.73 65.468) (end 136.588 65.468) (width 0.35) (layer F.Cu) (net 24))
 (segment (start 137.128 63.468) (end 137.16 63.5) (width 0.35) (layer F.Cu) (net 25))
 (segment (start 133.73 63.468) (end 137.128 63.468) (width 0.35) (layer F.Cu) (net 25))
 (via (at 128.778 63.5) (size 1) (layers F.Cu B.Cu) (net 25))
 (segment (start 128.778 63.5) (end 128.81 63.468) (width 0.35) (layer F.Cu) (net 25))
 (segment (start 128.81 63.468) (end 133.73 63.468) (width 0.35) (layer F.Cu) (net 25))
 (segment (start 125.73 63.5) (end 128.778 63.5) (width 0.35) (layer B.Cu) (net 25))
 (segment (start 136.652 61.468) (end 137.16 60.96) (width 0.35) (layer F.Cu) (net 26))
 (segment (start 133.73 61.468) (end 136.652 61.468) (width 0.35) (layer F.Cu) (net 26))
 (segment (start 136.112 59.468) (end 137.16 58.42) (width 0.35) (layer F.Cu) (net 27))
 (segment (start 133.73 59.468) (end 136.112 59.468) (width 0.35) (layer F.Cu) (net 27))
 (segment (start 135.572 57.468) (end 137.16 55.88) (width 0.35) (layer F.Cu) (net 28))
 (segment (start 133.73 57.468) (end 135.572 57.468) (width 0.35) (layer F.Cu) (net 28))
 (segment (start 128.016 56.642) (end 128.842 57.468) (width 0.35) (layer F.Cu) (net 28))
 (segment (start 128.842 57.468) (end 133.73 57.468) (width 0.35) (layer F.Cu) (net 28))
 (segment (start 128.016 42.926) (end 128.016 56.642) (width 0.35) (layer F.Cu) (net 28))
 (segment (start 133.73 54.23) (end 134.62 53.34) (width 0.35) (layer F.Cu) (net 29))
 (segment (start 134.62 53.34) (end 137.16 53.34) (width 0.35) (layer F.Cu) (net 29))
 (segment (start 133.73 55.468) (end 133.73 54.23) (width 0.35) (layer F.Cu) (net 29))
 (segment (start 125.476 54.61) (end 126.238 55.372) (width 0.35) (layer F.Cu) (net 29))
 (via (at 126.238 55.372) (size 1) (layers F.Cu B.Cu) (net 29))
 (segment (start 126.238 55.372) (end 130.048 55.372) (width 0.35) (layer B.Cu) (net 29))
 (via (at 130.048 55.372) (size 1) (layers F.Cu B.Cu) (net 29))
 (segment (start 130.048 55.372) (end 130.144 55.468) (width 0.35) (layer F.Cu) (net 29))
 (segment (start 130.144 55.468) (end 133.73 55.468) (width 0.35) (layer F.Cu) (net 29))
 (segment (start 125.476 42.926) (end 125.476 54.61) (width 0.35) (layer F.Cu) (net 29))
 (segment (start 124.968 61.468) (end 124.46 60.96) (width 0.35) (layer B.Cu) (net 30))
 (segment (start 124.46 60.96) (end 124.46 57.404) (width 0.35) (layer B.Cu) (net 30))
 (segment (start 128.186 61.468) (end 124.968 61.468) (width 0.35) (layer B.Cu) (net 30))
 (segment (start 125.476 57.404) (end 124.46 57.404) (width 0.35) (layer B.Cu) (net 30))
 (segment (start 127.17 57.404) (end 125.476 57.404) (width 0.35) (layer B.Cu) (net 30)))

